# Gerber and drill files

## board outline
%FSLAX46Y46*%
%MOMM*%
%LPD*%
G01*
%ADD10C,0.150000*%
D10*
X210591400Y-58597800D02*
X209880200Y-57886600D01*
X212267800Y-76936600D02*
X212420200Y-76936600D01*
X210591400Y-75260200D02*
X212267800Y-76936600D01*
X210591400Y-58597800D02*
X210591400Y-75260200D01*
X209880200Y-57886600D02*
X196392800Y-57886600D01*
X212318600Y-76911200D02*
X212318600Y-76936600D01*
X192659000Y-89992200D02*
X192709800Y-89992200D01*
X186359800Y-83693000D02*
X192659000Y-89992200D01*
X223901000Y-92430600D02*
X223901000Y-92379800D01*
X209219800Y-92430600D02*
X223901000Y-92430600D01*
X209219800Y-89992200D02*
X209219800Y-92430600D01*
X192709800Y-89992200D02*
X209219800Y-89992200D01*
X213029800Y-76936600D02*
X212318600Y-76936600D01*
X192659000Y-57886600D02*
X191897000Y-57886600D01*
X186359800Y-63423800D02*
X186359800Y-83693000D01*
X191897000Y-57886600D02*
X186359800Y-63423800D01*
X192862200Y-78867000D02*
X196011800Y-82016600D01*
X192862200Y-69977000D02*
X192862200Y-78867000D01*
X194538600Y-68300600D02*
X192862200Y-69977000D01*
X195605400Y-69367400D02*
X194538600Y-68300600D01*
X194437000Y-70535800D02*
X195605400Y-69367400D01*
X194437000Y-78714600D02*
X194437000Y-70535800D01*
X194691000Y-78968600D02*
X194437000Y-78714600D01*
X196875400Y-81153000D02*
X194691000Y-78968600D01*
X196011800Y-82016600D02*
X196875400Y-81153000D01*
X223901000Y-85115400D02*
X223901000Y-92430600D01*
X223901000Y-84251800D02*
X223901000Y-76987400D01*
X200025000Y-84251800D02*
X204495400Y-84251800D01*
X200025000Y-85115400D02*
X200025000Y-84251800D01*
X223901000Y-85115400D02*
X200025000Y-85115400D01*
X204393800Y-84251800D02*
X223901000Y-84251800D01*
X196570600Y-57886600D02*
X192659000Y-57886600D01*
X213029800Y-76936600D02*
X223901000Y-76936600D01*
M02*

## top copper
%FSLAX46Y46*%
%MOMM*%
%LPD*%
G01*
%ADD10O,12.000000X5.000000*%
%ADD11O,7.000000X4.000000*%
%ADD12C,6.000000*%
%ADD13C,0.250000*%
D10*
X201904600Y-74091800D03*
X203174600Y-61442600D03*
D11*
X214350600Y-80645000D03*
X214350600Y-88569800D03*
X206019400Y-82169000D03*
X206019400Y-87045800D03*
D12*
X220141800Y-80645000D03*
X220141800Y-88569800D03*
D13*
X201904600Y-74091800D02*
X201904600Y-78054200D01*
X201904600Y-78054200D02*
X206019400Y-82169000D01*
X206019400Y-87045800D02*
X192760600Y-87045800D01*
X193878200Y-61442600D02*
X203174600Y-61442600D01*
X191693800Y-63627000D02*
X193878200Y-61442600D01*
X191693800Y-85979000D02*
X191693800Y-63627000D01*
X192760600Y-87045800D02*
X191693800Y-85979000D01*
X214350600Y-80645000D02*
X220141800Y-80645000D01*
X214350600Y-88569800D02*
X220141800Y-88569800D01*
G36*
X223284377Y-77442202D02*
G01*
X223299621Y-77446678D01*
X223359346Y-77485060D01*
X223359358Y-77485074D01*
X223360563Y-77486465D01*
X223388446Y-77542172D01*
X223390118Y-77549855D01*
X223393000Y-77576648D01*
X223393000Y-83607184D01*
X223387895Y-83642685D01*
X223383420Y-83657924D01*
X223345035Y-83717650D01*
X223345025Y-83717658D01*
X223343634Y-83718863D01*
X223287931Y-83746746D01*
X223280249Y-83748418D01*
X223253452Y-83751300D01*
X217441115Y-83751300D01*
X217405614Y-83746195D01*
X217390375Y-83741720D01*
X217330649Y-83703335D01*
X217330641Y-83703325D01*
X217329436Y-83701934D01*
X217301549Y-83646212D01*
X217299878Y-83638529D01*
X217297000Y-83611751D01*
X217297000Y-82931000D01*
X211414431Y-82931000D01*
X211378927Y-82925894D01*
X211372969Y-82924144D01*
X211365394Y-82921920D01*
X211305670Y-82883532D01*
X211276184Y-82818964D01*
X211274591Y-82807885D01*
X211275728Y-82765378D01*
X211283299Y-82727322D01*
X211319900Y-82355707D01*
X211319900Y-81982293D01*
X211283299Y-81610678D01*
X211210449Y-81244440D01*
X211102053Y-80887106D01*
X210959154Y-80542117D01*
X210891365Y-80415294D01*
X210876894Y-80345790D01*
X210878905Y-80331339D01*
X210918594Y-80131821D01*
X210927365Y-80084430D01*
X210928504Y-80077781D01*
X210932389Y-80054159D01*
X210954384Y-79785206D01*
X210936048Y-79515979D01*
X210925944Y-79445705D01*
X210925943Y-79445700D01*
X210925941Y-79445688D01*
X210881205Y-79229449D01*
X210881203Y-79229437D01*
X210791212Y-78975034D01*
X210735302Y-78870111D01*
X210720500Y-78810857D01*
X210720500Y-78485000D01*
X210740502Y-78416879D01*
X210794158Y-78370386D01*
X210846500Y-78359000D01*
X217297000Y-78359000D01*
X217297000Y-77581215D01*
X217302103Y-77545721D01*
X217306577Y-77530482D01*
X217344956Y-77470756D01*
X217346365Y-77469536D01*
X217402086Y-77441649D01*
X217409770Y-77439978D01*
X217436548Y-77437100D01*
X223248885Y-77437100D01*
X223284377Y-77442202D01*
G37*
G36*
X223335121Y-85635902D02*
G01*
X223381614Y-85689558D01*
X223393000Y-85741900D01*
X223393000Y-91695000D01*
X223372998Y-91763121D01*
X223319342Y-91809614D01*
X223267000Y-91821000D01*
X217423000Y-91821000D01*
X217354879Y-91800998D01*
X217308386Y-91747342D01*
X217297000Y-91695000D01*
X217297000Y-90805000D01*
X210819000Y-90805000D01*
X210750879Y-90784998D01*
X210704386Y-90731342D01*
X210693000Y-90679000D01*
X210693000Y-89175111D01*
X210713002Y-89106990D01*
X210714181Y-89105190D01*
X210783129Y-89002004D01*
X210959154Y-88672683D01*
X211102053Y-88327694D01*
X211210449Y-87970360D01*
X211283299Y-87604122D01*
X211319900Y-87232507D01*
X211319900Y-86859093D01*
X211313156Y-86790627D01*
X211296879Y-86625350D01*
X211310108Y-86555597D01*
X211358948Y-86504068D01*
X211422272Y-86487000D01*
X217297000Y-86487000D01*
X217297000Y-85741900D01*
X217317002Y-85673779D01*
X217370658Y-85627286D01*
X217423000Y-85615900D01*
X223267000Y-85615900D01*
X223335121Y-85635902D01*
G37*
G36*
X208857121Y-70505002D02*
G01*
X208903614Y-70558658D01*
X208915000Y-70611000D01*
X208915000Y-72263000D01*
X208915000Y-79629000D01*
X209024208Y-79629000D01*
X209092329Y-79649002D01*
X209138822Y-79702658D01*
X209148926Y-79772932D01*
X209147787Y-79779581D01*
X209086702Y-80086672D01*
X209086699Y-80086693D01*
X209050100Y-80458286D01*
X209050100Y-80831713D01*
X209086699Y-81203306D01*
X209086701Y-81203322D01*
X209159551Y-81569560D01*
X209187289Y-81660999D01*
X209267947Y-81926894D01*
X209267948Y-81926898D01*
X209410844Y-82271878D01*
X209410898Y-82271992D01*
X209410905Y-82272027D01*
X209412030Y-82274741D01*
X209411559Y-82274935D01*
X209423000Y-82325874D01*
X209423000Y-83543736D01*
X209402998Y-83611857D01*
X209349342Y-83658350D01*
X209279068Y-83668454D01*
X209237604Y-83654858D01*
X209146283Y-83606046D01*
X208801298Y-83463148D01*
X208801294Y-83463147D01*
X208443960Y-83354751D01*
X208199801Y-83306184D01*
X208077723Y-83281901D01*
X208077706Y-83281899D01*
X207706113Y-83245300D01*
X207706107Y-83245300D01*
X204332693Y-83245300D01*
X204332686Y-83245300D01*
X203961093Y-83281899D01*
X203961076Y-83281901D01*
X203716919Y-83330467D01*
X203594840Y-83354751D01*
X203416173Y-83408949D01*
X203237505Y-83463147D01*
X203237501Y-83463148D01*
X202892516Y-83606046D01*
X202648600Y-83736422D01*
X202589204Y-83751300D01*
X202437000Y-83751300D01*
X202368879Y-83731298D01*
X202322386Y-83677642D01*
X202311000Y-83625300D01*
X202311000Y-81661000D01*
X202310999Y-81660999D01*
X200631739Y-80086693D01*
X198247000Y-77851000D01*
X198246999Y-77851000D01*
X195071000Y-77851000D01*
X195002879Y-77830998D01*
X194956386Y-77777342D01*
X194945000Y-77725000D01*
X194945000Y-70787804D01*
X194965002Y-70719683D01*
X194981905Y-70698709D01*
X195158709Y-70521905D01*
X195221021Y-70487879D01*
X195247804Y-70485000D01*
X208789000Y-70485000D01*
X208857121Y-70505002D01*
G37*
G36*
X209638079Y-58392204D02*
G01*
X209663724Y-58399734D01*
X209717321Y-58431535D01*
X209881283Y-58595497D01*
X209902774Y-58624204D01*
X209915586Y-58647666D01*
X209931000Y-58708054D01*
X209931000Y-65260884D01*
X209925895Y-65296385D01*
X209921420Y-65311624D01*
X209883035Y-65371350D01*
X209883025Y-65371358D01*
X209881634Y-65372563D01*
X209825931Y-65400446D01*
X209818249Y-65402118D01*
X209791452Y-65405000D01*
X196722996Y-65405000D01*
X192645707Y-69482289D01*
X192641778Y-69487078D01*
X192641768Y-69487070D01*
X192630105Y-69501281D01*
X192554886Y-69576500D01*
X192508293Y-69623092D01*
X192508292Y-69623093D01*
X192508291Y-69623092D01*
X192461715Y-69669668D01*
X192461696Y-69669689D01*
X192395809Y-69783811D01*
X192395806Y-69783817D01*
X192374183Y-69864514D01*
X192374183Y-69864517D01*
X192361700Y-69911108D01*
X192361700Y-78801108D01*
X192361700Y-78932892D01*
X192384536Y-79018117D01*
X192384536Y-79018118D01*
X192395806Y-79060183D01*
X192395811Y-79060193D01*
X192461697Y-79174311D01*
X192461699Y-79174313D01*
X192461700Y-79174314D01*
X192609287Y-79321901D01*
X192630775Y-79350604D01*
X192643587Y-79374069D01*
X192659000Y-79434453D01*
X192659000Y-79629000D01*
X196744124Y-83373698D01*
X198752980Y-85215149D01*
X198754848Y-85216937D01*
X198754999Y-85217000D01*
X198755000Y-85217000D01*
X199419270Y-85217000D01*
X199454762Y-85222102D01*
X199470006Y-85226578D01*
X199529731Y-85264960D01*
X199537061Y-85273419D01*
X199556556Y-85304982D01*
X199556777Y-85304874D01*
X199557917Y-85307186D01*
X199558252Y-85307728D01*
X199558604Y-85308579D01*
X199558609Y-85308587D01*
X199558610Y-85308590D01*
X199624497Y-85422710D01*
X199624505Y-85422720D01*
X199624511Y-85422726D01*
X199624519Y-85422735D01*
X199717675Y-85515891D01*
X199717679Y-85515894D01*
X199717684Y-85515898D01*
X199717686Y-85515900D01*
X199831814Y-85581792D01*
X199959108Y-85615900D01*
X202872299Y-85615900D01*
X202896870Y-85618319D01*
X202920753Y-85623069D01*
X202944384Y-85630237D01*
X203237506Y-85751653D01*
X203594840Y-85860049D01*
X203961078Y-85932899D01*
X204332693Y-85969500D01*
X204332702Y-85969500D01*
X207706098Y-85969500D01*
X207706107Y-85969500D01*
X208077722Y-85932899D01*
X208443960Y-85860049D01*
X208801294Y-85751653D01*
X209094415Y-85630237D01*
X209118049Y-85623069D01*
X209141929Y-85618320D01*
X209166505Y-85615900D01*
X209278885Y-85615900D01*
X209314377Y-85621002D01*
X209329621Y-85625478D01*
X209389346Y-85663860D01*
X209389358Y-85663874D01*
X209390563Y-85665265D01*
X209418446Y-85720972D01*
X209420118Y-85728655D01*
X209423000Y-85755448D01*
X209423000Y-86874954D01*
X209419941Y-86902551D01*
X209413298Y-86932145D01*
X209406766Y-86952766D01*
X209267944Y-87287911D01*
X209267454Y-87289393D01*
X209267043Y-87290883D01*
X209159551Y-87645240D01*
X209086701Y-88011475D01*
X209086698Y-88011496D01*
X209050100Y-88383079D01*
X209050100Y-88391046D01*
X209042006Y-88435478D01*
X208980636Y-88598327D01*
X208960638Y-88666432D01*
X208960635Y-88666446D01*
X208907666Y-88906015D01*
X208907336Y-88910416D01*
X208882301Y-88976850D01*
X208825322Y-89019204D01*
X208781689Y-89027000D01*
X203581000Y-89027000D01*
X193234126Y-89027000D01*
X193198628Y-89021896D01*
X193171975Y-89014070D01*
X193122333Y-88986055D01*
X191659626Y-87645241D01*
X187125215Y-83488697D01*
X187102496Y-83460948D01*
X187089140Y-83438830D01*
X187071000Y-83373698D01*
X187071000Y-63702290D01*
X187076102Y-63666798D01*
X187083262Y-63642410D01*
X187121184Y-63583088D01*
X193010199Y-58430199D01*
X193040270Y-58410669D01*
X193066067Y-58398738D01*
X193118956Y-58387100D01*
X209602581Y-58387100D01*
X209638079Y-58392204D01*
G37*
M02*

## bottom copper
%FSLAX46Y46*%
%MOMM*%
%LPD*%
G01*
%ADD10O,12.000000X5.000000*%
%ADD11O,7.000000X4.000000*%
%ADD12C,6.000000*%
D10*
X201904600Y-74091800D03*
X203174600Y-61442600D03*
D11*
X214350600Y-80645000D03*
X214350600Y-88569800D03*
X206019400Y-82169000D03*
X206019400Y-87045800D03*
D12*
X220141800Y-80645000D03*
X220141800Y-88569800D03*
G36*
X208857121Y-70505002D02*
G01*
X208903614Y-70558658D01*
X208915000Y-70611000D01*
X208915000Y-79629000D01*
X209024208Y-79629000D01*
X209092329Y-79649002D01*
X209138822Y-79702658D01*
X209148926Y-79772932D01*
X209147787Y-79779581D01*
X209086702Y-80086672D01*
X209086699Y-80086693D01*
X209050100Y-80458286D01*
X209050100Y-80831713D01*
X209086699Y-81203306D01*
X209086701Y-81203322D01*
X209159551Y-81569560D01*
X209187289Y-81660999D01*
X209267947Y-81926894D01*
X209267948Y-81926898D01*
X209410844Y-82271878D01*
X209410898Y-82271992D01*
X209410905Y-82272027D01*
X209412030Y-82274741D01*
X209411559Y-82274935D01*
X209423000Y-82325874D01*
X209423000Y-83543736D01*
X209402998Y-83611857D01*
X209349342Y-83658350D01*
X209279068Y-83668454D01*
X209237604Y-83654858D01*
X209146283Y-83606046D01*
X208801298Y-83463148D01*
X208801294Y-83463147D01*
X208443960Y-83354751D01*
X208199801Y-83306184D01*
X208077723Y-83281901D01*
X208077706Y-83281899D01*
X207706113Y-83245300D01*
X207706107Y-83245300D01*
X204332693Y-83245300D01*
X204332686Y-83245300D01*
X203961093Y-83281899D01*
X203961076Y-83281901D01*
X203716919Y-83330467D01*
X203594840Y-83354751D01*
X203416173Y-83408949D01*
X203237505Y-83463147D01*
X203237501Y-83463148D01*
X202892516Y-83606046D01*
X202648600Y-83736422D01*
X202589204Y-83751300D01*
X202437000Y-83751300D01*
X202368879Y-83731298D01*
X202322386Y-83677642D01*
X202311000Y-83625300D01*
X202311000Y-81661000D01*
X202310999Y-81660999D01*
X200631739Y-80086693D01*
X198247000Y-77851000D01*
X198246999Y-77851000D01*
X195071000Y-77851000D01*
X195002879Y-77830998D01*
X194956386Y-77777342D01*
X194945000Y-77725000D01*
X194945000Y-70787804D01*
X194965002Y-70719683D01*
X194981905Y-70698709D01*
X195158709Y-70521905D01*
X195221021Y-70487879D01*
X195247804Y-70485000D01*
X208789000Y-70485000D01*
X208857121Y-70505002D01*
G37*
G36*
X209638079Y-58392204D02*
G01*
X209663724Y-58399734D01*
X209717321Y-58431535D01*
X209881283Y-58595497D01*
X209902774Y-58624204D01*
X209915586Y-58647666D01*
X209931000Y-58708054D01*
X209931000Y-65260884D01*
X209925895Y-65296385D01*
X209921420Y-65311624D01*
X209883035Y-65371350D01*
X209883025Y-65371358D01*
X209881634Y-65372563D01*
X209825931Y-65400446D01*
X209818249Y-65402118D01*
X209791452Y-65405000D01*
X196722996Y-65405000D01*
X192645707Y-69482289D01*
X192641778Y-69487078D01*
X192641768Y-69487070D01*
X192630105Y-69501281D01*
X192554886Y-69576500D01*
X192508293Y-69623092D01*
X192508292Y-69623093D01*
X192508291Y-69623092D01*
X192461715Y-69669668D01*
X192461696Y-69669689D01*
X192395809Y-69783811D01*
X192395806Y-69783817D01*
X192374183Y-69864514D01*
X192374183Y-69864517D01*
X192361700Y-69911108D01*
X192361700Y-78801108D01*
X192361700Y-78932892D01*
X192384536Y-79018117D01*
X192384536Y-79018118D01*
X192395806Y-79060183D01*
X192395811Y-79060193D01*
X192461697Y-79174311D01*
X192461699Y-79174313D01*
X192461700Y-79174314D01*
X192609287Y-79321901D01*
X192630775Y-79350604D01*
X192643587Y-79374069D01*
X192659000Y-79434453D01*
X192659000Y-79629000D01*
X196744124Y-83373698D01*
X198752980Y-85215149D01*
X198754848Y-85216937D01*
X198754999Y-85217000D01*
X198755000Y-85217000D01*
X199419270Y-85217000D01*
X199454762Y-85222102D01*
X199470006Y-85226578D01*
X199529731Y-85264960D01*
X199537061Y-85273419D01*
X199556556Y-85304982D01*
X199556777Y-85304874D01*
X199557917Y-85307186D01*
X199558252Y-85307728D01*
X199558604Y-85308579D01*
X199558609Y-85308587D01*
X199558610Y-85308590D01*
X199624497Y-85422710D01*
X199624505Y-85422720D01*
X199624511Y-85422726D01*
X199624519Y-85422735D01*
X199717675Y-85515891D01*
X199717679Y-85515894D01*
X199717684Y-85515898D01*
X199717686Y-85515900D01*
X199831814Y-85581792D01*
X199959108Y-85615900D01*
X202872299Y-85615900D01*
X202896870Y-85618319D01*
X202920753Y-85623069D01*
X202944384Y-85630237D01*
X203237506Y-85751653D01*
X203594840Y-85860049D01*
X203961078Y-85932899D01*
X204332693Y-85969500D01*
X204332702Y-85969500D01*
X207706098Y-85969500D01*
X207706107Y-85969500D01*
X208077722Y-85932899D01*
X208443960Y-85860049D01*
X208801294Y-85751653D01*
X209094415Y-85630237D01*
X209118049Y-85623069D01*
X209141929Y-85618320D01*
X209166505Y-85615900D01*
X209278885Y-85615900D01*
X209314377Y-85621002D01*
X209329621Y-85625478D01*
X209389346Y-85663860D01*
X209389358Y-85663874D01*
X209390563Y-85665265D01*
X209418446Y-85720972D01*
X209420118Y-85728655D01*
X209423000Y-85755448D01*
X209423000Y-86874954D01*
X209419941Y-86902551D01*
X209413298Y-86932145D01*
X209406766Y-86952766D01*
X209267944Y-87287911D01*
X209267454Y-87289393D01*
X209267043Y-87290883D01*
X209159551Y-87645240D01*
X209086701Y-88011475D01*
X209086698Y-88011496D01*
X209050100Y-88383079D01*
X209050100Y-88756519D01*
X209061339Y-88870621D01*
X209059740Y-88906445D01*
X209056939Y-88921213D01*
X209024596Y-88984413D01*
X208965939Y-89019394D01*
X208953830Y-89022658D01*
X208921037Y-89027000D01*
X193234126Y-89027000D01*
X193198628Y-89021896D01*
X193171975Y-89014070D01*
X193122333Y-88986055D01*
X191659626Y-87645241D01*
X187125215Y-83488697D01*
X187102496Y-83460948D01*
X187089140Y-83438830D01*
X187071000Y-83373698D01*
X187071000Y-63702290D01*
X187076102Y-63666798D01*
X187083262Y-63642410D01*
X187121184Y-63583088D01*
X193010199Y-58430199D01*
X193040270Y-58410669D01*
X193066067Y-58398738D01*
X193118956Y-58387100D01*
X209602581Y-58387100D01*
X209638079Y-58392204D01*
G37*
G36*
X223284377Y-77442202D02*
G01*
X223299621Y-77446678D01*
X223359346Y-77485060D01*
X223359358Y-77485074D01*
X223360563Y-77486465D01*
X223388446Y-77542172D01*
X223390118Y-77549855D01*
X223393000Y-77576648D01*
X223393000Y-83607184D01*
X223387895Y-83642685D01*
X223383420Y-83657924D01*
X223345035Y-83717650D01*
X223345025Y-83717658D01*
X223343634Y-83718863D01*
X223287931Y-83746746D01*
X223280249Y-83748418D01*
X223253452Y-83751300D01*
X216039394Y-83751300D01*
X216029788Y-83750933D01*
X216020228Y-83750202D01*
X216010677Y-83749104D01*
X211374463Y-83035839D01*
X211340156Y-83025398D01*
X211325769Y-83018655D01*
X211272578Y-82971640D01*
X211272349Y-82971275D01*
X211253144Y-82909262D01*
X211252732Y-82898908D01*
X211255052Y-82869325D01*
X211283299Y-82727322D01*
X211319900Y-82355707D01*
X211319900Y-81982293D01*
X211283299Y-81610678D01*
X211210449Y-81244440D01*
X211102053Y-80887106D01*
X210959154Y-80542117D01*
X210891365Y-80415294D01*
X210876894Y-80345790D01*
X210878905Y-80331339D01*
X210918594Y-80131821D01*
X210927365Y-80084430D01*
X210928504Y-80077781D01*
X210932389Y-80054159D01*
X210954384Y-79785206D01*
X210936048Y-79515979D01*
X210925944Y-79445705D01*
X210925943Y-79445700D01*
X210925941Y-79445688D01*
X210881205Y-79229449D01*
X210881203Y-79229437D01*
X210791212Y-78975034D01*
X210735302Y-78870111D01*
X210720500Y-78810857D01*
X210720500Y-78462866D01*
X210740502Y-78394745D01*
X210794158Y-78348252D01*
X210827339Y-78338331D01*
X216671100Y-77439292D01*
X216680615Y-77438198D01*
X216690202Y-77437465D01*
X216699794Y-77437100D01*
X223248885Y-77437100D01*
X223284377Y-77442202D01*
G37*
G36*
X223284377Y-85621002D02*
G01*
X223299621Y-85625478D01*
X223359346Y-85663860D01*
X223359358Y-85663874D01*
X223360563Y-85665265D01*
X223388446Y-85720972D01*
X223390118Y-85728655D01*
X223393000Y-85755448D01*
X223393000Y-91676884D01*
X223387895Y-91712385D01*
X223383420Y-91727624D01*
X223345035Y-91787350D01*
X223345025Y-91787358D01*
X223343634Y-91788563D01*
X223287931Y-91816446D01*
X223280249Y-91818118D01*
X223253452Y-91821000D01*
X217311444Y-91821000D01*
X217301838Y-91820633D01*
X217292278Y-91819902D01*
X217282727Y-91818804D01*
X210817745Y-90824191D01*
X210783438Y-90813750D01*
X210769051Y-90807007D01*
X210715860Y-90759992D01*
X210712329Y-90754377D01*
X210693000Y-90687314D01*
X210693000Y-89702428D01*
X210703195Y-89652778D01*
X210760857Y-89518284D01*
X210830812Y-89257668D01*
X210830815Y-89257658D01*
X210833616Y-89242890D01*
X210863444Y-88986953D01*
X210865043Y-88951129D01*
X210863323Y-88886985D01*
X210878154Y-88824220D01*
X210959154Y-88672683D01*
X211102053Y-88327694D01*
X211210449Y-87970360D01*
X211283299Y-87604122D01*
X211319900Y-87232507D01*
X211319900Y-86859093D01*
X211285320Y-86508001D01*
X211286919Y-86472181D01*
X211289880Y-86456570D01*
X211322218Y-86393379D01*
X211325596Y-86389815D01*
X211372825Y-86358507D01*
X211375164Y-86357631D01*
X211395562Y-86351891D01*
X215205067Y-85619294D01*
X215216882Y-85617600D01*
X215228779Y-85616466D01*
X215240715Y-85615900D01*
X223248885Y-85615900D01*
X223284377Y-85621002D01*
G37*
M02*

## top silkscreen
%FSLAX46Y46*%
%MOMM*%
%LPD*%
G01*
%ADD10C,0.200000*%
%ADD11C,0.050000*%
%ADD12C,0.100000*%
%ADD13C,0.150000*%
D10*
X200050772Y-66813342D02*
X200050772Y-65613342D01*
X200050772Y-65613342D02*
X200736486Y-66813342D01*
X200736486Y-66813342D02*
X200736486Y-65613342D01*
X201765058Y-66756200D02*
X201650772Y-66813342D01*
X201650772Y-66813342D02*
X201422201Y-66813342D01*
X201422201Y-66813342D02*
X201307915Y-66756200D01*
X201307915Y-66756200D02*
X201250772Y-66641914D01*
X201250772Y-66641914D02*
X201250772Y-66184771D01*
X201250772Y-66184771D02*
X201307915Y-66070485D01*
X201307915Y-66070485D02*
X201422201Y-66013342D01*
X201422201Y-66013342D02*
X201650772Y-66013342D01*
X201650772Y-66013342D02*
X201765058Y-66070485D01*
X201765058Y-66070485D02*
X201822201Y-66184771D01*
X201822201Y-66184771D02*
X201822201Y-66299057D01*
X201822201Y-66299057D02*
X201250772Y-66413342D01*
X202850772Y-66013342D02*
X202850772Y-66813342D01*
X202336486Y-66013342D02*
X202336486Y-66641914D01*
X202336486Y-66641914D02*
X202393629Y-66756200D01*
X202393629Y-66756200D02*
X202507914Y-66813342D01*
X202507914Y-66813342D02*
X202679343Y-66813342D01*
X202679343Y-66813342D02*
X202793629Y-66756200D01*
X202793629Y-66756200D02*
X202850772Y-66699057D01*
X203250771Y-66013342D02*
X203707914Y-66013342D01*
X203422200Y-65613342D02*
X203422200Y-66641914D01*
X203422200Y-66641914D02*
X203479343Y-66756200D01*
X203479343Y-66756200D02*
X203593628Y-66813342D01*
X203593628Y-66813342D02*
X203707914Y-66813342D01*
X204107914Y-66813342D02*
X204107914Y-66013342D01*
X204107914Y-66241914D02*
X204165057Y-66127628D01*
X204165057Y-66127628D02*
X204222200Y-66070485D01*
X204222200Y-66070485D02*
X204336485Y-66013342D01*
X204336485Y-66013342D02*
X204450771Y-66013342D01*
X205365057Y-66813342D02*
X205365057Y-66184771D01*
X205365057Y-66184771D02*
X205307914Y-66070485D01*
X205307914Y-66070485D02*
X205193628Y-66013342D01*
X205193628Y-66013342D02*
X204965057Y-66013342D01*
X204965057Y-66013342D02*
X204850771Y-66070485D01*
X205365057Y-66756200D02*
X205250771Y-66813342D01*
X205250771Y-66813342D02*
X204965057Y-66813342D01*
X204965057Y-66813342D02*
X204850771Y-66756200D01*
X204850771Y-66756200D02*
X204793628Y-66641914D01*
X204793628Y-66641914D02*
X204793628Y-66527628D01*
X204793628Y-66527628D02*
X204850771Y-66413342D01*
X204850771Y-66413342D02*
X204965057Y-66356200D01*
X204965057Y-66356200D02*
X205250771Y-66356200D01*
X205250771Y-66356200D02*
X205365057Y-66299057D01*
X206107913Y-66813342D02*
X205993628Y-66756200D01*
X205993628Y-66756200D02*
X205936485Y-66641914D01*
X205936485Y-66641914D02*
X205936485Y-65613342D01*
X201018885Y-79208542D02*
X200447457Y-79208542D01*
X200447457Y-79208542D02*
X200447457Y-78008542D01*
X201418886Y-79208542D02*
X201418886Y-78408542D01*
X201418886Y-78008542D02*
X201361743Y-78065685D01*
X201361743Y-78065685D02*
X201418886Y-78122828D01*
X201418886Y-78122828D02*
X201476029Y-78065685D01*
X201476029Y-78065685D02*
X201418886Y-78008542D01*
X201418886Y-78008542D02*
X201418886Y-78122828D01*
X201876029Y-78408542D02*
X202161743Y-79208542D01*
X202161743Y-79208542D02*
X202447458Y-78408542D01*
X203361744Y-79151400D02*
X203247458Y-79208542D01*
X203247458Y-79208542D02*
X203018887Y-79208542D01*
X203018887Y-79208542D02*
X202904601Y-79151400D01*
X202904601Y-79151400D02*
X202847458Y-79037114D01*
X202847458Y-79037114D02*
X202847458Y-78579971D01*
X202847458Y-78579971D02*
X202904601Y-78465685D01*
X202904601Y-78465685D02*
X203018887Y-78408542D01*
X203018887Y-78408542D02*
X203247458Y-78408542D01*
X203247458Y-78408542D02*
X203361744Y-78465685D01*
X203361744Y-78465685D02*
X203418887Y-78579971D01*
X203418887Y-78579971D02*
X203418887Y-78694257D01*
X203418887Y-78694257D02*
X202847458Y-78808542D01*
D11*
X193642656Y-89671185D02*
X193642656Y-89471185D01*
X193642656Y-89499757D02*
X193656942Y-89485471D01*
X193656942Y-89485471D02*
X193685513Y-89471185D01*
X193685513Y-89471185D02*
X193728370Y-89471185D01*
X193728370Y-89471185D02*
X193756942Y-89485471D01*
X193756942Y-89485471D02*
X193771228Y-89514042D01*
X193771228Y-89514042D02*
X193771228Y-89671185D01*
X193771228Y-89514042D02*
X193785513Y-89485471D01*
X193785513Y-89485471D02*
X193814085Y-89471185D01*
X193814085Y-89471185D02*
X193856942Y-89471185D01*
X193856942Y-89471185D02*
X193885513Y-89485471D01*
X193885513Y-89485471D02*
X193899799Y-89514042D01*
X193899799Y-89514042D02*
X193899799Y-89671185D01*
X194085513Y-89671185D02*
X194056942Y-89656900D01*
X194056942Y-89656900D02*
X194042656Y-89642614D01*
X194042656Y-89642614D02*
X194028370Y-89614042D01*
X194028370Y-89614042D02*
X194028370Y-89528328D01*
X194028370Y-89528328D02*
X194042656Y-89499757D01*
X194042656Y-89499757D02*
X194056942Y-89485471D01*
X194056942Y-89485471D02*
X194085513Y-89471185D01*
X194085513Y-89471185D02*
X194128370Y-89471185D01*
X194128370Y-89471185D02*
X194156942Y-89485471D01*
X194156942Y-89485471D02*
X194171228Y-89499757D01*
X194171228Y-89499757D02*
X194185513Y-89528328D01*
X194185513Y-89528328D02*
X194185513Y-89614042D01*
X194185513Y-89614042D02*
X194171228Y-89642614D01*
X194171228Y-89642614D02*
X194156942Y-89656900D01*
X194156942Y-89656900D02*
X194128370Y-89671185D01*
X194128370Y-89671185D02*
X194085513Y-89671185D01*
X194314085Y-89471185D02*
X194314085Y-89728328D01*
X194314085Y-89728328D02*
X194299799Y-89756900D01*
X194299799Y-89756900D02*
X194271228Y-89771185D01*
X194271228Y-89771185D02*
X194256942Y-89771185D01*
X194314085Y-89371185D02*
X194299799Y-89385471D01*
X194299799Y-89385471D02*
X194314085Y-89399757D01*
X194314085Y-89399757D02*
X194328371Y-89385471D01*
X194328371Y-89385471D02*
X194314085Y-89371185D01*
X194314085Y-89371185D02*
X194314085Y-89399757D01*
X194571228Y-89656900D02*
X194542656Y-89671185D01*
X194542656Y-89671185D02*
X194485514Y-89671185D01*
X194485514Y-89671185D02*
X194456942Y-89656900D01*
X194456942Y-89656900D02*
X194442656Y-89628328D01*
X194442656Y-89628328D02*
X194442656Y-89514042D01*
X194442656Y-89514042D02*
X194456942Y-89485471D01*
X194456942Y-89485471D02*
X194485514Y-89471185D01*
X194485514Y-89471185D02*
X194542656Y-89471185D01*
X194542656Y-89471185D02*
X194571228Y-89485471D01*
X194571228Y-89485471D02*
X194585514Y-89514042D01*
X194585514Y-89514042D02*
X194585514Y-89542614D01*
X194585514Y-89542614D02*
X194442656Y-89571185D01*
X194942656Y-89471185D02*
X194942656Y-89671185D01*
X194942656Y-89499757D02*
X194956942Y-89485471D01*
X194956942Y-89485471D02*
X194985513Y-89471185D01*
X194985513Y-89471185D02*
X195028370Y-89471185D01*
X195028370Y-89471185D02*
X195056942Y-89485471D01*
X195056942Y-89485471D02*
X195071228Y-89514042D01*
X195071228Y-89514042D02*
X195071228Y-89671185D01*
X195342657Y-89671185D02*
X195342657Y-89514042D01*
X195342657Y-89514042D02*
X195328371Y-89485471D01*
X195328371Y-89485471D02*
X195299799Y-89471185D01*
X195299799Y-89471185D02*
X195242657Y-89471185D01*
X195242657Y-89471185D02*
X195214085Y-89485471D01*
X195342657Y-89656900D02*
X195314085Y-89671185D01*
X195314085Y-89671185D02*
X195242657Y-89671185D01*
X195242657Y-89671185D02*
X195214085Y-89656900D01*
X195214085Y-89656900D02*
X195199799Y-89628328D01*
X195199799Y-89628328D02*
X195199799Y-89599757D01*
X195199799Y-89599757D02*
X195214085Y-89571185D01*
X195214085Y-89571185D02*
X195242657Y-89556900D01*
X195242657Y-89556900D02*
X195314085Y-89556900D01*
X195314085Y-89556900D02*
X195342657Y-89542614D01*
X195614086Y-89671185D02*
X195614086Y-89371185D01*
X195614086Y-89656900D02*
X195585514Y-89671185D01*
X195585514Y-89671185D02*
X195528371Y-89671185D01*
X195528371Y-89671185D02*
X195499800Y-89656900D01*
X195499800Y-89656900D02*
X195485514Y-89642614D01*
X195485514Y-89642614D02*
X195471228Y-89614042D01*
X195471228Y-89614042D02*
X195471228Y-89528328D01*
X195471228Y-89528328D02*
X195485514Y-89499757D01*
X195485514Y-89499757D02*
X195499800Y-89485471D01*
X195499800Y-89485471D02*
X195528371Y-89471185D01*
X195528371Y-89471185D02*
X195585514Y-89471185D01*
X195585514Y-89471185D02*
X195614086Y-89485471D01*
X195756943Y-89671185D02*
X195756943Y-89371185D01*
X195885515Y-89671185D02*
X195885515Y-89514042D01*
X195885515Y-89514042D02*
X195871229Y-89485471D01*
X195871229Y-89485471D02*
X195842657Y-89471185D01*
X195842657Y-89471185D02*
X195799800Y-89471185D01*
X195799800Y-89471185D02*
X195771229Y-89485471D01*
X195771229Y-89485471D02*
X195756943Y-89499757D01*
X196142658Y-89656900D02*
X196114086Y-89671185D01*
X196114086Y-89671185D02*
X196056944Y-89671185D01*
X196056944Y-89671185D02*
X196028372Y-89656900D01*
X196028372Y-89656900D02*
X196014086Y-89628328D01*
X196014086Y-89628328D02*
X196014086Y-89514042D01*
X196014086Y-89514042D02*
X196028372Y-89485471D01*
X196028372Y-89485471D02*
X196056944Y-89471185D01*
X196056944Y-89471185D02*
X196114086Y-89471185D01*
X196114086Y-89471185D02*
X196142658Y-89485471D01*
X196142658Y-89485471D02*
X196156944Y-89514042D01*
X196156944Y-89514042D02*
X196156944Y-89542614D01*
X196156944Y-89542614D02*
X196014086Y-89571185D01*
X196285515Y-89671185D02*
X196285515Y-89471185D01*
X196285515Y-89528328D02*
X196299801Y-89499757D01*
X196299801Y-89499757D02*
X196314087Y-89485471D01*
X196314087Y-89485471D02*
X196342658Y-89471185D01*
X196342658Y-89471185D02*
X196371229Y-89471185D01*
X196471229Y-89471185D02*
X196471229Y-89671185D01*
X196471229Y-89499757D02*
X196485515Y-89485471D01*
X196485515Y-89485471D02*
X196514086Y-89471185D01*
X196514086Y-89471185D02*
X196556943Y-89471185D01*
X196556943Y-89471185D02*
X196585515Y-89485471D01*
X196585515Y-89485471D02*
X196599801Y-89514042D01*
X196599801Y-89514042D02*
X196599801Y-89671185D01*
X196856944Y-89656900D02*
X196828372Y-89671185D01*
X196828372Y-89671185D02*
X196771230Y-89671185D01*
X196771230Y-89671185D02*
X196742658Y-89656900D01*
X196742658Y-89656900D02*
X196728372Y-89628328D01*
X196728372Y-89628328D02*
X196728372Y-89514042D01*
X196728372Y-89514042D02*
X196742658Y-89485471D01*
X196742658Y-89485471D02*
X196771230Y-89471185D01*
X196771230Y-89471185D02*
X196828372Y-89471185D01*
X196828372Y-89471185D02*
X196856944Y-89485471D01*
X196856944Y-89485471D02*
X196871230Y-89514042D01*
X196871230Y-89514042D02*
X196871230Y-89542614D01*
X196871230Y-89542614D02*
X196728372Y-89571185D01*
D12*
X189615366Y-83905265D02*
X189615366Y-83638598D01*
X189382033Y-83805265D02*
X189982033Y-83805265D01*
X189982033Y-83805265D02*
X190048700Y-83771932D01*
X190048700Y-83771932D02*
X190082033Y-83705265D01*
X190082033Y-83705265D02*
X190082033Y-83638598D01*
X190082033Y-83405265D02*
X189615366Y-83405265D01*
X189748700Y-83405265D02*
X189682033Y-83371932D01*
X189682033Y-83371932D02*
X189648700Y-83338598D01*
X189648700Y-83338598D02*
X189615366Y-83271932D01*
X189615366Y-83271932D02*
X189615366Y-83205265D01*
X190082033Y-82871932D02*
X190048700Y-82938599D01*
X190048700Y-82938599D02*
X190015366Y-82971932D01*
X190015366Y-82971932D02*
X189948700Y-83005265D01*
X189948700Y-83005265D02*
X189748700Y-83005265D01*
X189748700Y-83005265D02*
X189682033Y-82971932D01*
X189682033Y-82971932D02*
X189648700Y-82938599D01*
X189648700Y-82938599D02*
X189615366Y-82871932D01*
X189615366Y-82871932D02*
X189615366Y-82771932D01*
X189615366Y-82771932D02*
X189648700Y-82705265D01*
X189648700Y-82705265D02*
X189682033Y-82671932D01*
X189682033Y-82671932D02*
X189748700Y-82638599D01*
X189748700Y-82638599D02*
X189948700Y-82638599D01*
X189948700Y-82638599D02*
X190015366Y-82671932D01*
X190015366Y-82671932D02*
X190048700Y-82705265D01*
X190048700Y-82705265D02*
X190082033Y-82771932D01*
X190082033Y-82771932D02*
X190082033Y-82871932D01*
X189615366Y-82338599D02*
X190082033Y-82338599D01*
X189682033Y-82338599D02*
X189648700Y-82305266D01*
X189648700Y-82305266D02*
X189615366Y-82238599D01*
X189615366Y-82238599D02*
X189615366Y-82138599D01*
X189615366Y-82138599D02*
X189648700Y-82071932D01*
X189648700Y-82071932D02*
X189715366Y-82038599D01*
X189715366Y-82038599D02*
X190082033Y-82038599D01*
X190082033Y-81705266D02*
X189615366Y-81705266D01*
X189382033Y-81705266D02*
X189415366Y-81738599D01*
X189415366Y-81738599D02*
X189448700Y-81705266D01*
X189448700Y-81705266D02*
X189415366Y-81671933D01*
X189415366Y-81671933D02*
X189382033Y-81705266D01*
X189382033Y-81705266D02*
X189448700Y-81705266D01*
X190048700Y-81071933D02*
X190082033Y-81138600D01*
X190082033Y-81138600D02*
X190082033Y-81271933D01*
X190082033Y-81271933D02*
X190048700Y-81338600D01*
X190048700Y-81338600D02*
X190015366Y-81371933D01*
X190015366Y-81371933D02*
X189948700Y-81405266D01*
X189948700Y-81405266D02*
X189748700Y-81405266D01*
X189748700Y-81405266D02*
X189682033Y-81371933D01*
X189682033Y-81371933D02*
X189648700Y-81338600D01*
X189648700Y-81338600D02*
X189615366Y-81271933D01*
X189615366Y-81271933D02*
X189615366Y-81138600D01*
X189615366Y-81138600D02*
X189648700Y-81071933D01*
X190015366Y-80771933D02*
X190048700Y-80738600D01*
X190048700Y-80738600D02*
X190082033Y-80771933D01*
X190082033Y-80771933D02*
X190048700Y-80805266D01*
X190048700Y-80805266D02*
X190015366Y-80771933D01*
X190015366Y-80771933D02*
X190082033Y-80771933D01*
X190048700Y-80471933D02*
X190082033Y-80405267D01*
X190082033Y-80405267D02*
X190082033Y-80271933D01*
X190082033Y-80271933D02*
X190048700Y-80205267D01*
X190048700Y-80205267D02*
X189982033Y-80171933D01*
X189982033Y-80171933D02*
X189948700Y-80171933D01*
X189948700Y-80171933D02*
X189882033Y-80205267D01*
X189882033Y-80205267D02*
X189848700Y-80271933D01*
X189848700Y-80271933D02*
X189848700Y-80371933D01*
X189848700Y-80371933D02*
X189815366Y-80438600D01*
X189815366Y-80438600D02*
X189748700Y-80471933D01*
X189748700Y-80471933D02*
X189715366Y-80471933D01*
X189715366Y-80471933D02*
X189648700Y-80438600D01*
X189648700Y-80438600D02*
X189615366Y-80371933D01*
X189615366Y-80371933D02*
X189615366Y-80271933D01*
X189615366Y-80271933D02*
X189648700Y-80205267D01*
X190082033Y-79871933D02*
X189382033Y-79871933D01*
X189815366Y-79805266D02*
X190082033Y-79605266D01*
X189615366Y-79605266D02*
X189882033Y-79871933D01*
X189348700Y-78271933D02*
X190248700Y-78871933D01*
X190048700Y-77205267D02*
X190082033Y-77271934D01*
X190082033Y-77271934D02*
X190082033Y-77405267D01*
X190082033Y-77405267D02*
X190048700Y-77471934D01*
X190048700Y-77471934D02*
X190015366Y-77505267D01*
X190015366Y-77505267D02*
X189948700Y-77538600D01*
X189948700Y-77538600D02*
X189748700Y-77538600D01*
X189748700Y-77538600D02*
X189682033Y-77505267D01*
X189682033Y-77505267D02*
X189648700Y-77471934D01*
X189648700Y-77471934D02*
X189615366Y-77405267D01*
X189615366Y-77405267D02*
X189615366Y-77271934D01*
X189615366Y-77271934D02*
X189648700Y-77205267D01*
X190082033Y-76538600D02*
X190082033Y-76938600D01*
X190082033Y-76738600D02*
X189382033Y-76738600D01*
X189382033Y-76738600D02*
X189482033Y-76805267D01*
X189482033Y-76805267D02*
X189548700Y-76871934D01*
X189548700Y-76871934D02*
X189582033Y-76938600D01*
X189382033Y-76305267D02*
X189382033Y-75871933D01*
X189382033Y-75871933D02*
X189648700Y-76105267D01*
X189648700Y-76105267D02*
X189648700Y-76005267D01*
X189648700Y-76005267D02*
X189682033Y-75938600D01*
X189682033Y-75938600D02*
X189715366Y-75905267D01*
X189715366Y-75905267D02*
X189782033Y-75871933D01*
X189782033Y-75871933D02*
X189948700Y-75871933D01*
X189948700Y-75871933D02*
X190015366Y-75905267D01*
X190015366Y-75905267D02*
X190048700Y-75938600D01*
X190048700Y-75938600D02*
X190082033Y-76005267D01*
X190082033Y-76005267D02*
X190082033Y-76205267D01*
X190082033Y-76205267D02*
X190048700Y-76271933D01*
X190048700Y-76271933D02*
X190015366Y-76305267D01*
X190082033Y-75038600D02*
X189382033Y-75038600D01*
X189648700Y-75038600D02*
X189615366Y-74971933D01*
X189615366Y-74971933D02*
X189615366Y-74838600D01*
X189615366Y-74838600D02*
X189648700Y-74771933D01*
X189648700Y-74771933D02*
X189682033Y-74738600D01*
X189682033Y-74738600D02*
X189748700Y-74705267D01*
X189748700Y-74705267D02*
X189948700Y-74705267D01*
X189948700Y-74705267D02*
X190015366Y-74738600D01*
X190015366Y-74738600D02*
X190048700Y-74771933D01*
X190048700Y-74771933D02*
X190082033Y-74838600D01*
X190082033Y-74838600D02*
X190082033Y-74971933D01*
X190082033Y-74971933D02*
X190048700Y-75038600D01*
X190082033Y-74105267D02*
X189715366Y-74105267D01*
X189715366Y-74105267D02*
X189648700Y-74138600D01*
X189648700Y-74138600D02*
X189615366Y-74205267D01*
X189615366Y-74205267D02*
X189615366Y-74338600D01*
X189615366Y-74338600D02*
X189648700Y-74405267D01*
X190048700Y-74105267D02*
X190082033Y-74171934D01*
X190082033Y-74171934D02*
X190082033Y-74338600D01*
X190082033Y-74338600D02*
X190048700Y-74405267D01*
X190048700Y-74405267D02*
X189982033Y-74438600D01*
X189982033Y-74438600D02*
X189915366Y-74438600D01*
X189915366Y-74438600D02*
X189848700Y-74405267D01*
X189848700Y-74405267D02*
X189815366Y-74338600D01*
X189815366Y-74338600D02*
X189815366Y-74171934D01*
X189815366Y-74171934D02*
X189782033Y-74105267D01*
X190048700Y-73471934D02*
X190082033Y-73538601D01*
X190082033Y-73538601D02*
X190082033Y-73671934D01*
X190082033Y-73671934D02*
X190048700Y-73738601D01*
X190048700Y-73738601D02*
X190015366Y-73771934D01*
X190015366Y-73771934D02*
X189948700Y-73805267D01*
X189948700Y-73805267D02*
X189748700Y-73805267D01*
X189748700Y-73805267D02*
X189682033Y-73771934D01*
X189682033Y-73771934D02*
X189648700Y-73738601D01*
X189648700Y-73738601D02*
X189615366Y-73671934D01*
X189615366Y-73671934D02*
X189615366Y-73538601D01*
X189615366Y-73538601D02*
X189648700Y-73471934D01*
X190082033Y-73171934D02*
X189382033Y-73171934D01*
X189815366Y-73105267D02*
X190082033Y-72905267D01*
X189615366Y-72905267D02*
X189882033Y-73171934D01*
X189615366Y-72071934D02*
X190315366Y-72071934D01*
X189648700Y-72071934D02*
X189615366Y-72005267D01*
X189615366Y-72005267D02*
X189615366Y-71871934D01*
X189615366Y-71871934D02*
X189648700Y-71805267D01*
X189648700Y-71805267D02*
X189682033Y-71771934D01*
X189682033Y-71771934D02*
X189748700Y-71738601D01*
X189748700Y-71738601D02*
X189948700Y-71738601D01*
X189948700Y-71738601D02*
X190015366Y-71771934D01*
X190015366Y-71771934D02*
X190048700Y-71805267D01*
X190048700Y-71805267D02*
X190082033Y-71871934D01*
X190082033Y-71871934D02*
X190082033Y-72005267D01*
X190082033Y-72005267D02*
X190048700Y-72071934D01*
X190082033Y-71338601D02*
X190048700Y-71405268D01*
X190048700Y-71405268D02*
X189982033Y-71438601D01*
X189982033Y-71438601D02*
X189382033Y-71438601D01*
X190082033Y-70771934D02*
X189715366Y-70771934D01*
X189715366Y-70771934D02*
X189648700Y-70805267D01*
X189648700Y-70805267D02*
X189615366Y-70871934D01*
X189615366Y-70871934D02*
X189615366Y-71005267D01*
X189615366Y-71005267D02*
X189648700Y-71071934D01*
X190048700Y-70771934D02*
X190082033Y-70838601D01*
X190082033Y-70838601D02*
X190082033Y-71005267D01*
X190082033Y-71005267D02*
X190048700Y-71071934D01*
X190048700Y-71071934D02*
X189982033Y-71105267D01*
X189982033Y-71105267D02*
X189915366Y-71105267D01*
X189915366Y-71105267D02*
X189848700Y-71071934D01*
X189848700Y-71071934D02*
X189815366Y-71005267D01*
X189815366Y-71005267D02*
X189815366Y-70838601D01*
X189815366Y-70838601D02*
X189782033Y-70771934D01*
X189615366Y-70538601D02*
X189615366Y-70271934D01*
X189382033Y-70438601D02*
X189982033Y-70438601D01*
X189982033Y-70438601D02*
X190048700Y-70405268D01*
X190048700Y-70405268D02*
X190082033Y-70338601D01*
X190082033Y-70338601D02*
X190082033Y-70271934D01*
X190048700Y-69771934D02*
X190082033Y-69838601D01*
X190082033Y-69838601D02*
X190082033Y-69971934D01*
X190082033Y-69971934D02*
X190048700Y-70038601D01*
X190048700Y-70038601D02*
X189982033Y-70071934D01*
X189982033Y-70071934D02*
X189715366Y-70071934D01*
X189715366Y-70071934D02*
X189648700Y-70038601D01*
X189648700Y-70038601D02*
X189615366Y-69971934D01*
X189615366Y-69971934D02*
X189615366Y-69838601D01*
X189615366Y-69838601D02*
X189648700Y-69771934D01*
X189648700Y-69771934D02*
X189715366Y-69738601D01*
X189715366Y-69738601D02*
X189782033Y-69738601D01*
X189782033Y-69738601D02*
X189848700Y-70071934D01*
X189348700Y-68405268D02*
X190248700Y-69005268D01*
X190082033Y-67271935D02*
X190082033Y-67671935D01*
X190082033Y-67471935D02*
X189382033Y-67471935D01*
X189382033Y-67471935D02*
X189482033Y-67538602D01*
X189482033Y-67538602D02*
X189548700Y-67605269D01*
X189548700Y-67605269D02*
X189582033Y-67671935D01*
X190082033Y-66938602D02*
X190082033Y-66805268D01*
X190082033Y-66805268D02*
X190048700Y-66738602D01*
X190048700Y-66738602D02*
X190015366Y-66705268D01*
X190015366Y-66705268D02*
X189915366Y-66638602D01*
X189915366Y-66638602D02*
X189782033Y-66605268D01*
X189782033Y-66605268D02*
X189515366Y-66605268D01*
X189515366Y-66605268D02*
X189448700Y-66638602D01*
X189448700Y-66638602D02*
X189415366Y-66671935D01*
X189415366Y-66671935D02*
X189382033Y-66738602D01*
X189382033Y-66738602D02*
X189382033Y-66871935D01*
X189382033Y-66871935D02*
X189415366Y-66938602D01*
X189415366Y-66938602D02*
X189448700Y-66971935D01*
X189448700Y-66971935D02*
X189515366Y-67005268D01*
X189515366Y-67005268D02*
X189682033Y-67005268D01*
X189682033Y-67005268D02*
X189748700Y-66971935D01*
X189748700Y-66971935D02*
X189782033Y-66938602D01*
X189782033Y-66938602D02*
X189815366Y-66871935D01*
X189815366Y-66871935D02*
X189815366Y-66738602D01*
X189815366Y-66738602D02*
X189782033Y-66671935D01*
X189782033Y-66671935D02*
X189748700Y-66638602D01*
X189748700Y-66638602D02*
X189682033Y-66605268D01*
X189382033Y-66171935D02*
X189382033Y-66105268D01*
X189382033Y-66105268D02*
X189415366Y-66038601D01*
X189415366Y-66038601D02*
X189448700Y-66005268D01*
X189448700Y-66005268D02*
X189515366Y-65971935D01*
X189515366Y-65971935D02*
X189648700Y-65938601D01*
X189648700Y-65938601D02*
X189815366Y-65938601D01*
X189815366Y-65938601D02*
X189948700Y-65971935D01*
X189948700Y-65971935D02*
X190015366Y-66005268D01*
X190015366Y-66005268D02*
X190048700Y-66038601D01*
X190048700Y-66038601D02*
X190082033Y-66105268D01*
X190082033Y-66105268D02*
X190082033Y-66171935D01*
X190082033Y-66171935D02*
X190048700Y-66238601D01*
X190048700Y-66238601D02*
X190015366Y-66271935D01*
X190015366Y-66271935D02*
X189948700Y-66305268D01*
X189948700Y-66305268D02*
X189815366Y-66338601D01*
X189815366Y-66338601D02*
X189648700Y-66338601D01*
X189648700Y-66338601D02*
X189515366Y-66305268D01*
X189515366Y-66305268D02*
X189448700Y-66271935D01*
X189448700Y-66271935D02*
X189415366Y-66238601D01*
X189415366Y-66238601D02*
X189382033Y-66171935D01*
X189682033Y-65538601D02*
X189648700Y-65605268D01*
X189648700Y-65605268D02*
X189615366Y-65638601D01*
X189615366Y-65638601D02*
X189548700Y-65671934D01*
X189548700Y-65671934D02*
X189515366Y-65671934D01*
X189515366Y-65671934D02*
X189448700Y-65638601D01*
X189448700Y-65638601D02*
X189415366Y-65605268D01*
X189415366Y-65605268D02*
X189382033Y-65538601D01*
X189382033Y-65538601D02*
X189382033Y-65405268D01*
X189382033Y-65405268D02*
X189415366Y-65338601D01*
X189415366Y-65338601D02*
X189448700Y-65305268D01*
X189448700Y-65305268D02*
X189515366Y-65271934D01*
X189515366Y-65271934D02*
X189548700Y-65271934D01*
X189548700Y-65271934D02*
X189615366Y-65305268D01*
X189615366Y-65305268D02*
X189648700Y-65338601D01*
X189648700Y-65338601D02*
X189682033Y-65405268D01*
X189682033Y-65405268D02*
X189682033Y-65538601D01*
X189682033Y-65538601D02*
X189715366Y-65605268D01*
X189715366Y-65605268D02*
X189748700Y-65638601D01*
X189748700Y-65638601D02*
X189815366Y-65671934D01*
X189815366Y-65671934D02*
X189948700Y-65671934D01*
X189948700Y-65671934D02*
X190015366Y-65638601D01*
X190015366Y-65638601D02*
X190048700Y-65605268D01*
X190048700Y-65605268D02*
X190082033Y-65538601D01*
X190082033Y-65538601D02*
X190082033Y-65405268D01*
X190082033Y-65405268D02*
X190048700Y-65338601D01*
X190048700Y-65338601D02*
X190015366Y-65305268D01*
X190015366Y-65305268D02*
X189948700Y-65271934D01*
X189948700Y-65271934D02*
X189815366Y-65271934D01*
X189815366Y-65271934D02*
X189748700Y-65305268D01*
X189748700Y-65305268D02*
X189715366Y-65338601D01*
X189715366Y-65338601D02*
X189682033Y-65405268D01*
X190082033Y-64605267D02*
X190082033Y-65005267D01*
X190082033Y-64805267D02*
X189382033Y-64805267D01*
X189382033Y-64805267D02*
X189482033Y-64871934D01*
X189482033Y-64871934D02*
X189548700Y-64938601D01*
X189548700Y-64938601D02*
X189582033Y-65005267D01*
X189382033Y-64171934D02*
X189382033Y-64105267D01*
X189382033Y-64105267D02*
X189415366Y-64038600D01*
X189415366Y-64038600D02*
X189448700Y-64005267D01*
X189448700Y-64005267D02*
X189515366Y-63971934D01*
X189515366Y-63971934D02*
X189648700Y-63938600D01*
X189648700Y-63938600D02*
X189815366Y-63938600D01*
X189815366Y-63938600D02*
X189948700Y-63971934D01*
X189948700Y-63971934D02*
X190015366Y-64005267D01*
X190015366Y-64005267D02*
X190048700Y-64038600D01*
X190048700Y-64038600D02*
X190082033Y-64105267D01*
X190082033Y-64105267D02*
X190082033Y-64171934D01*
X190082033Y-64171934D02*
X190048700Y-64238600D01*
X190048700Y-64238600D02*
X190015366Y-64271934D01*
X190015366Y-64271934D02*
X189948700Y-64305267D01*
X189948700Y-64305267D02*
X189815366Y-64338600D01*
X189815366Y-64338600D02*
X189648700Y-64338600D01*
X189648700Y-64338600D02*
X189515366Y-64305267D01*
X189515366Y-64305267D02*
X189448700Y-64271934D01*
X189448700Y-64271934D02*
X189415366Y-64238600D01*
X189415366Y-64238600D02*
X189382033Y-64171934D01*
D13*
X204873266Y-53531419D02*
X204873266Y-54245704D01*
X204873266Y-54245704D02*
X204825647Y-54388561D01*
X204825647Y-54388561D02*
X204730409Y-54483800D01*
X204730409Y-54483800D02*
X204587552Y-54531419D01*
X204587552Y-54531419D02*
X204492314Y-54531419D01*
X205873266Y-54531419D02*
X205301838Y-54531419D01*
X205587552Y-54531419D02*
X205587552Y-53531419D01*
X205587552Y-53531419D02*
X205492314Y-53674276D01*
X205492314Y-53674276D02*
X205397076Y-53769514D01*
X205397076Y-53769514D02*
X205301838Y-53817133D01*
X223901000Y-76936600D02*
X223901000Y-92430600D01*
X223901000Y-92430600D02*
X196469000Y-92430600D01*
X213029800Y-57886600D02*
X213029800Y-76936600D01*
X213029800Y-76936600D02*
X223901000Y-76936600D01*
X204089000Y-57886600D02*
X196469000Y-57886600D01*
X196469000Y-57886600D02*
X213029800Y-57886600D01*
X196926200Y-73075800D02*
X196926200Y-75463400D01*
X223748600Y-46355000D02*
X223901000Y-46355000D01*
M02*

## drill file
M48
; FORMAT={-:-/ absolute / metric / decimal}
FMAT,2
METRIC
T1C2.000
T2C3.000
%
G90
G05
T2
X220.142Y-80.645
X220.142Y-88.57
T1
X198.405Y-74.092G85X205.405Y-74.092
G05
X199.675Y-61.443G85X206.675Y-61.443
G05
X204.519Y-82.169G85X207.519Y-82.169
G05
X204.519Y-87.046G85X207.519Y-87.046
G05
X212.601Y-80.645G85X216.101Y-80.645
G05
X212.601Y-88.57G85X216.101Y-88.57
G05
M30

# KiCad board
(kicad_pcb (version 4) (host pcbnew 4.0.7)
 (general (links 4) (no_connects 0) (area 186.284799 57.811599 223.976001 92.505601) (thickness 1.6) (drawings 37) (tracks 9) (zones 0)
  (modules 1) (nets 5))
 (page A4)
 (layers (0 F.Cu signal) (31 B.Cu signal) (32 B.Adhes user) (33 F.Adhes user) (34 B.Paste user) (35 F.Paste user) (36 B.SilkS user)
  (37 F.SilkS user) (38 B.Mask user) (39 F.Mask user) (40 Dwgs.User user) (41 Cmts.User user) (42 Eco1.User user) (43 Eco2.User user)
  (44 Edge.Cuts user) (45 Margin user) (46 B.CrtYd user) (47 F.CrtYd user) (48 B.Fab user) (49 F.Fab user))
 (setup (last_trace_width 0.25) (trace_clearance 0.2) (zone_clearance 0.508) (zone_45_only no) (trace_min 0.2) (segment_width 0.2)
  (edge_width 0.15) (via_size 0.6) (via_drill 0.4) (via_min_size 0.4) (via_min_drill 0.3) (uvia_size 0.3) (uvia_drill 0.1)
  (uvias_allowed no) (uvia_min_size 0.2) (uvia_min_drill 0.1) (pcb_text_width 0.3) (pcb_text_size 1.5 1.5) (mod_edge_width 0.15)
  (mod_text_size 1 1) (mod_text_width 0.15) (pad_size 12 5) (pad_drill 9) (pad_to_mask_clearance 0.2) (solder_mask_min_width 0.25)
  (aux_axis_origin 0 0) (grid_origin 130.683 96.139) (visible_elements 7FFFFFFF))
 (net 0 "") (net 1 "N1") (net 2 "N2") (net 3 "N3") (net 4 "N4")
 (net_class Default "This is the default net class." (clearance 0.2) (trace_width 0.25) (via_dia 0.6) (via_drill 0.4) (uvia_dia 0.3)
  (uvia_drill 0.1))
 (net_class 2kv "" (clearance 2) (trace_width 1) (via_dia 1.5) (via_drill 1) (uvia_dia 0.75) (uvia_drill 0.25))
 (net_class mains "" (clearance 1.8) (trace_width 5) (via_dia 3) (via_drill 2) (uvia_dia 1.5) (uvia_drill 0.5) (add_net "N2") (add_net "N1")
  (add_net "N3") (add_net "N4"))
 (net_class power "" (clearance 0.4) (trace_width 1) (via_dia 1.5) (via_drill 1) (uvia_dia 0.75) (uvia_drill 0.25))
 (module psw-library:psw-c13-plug (layer F.Cu) (at 196.469 46.355)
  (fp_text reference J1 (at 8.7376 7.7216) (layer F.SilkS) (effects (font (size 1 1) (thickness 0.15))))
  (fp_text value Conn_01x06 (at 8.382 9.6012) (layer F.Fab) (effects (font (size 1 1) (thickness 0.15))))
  (fp_line (start 27.432 30.5816) (end 27.432 46.0756) (layer F.SilkS) (width 0.15))
  (fp_line (start 27.432 46.0756) (end 0 46.0756) (layer F.SilkS) (width 0.15))
  (fp_line (start 16.5608 11.5316) (end 16.5608 30.5816) (layer F.SilkS) (width 0.15))
  (fp_line (start 16.5608 30.5816) (end 27.432 30.5816) (layer F.SilkS) (width 0.15))
  (fp_line (start 7.62 11.5316) (end 0 11.5316) (layer F.SilkS) (width 0.15))
  (fp_line (start 0 11.5316) (end 16.5608 11.5316) (layer F.SilkS) (width 0.15))
  (fp_line (start 0.4572 26.7208) (end 0.4572 29.1084) (layer F.SilkS) (width 0.15))
  (fp_line (start 27.2796 0) (end 27.432 0) (layer F.SilkS) (width 0.15))
  (pad 2 thru_hole oval (at 5.4356 27.7368) (size 12 5) (drill oval 9 2) (layers *.Cu *.Mask) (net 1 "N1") (zone_connect 2))
  (pad 1 thru_hole oval (at 6.7056 15.0876) (size 12 5) (drill oval 9 2) (layers *.Cu *.Mask) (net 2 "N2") (zone_connect 2))
  (pad 5 thru_hole oval (at 17.8816 34.29) (size 7 4) (drill oval 5.5 2) (layers *.Cu *.Mask) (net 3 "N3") (zone_connect 2))
  (pad 6 thru_hole oval (at 17.8816 42.2148) (size 7 4) (drill oval 5.5 2) (layers *.Cu *.Mask) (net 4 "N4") (zone_connect 2))
  (pad 3 thru_hole oval (at 9.5504 35.814) (size 7 4) (drill oval 5 2) (layers *.Cu *.Mask) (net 1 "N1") (zone_connect 2))
  (pad 4 thru_hole oval (at 9.5504 40.6908) (size 7 4) (drill oval 5 2) (layers *.Cu *.Mask) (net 2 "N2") (zone_connect 2))
  (pad 5 thru_hole circle (at 23.6728 34.29) (size 6 6) (drill 3) (layers *.Cu *.Mask) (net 3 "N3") (zone_connect 2))
  (pad 6 thru_hole circle (at 23.6728 42.2148) (size 6 6) (drill 3) (layers *.Cu *.Mask) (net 4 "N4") (zone_connect 2)))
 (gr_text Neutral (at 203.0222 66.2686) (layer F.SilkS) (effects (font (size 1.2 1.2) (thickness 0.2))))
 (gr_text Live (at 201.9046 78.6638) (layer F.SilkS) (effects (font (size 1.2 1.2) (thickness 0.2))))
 (gr_line (start 210.5914 58.5978) (end 209.8802 57.8866) (angle 90) (layer Edge.Cuts) (width 0.15))
 (gr_line (start 212.2678 76.9366) (end 212.4202 76.9366) (angle 90) (layer Edge.Cuts) (width 0.15))
 (gr_line (start 210.5914 75.2602) (end 212.2678 76.9366) (angle 90) (layer Edge.Cuts) (width 0.15))
 (gr_line (start 210.5914 58.5978) (end 210.5914 75.2602) (angle 90) (layer Edge.Cuts) (width 0.15))
 (gr_line (start 209.8802 57.8866) (end 196.3928 57.8866) (angle 90) (layer Edge.Cuts) (width 0.15))
 (gr_line (start 212.3186 76.9112) (end 212.3186 76.9366) (angle 90) (layer Edge.Cuts) (width 0.15))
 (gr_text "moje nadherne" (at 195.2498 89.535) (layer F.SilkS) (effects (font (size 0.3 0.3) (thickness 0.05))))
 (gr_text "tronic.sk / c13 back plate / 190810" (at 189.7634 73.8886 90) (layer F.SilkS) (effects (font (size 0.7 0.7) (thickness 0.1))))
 (gr_line (start 192.659 89.9922) (end 192.7098 89.9922) (angle 90) (layer Edge.Cuts) (width 0.15))
 (gr_line (start 186.3598 83.693) (end 192.659 89.9922) (angle 90) (layer Edge.Cuts) (width 0.15))
 (gr_line (start 223.901 92.4306) (end 223.901 92.3798) (angle 90) (layer Edge.Cuts) (width 0.15))
 (gr_line (start 209.2198 92.4306) (end 223.901 92.4306) (angle 90) (layer Edge.Cuts) (width 0.15))
 (gr_line (start 209.2198 89.9922) (end 209.2198 92.4306) (angle 90) (layer Edge.Cuts) (width 0.15))
 (gr_line (start 192.7098 89.9922) (end 209.2198 89.9922) (angle 90) (layer Edge.Cuts) (width 0.15))
 (gr_line (start 213.0298 76.9366) (end 212.3186 76.9366) (angle 90) (layer Edge.Cuts) (width 0.15))
 (gr_line (start 192.659 57.8866) (end 191.897 57.8866) (angle 90) (layer Edge.Cuts) (width 0.15))
 (gr_line (start 186.3598 63.4238) (end 186.3598 83.693) (angle 90) (layer Edge.Cuts) (width 0.15))
 (gr_line (start 191.897 57.8866) (end 186.3598 63.4238) (angle 90) (layer Edge.Cuts) (width 0.15))
 (gr_line (start 192.8622 78.867) (end 196.0118 82.0166) (angle 90) (layer Edge.Cuts) (width 0.15))
 (gr_line (start 192.8622 69.977) (end 192.8622 78.867) (angle 90) (layer Edge.Cuts) (width 0.15))
 (gr_line (start 194.5386 68.3006) (end 192.8622 69.977) (angle 90) (layer Edge.Cuts) (width 0.15))
 (gr_line (start 195.6054 69.3674) (end 194.5386 68.3006) (angle 90) (layer Edge.Cuts) (width 0.15))
 (gr_line (start 194.437 70.5358) (end 195.6054 69.3674) (angle 90) (layer Edge.Cuts) (width 0.15))
 (gr_line (start 194.437 78.7146) (end 194.437 70.5358) (angle 90) (layer Edge.Cuts) (width 0.15))
 (gr_line (start 194.691 78.9686) (end 194.437 78.7146) (angle 90) (layer Edge.Cuts) (width 0.15))
 (gr_line (start 196.8754 81.153) (end 194.691 78.9686) (angle 90) (layer Edge.Cuts) (width 0.15))
 (gr_line (start 196.0118 82.0166) (end 196.8754 81.153) (angle 90) (layer Edge.Cuts) (width 0.15))
 (gr_line (start 223.901 85.1154) (end 223.901 92.4306) (angle 90) (layer Edge.Cuts) (width 0.15))
 (gr_line (start 223.901 84.2518) (end 223.901 76.9874) (angle 90) (layer Edge.Cuts) (width 0.15))
 (gr_line (start 200.025 84.2518) (end 204.4954 84.2518) (angle 90) (layer Edge.Cuts) (width 0.15))
 (gr_line (start 200.025 85.1154) (end 200.025 84.2518) (angle 90) (layer Edge.Cuts) (width 0.15))
 (gr_line (start 223.901 85.1154) (end 200.025 85.1154) (angle 90) (layer Edge.Cuts) (width 0.15))
 (gr_line (start 204.3938 84.2518) (end 223.901 84.2518) (angle 90) (layer Edge.Cuts) (width 0.15))
 (gr_line (start 196.5706 57.8866) (end 192.659 57.8866) (angle 90) (layer Edge.Cuts) (width 0.15))
 (gr_line (start 213.0298 76.9366) (end 223.901 76.9366) (angle 90) (layer Edge.Cuts) (width 0.15))
 (segment (start 201.9046 74.0918) (end 201.9046 78.0542) (width 0.25) (layer F.Cu) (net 1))
 (segment (start 201.9046 78.0542) (end 206.0194 82.169) (width 0.25) (layer F.Cu) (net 1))
 (segment (start 206.0194 87.0458) (end 192.7606 87.0458) (width 0.25) (layer F.Cu) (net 2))
 (segment (start 193.8782 61.4426) (end 203.1746 61.4426) (width 0.25) (layer F.Cu) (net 2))
 (segment (start 191.6938 63.627) (end 193.8782 61.4426) (width 0.25) (layer F.Cu) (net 2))
 (segment (start 191.6938 85.979) (end 191.6938 63.627) (width 0.25) (layer F.Cu) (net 2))
 (segment (start 192.7606 87.0458) (end 191.6938 85.979) (width 0.25) (layer F.Cu) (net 2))
 (segment (start 214.3506 80.645) (end 220.1418 80.645) (width 0.25) (layer F.Cu) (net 3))
 (segment (start 214.3506 88.5698) (end 220.1418 88.5698) (width 0.25) (layer F.Cu) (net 4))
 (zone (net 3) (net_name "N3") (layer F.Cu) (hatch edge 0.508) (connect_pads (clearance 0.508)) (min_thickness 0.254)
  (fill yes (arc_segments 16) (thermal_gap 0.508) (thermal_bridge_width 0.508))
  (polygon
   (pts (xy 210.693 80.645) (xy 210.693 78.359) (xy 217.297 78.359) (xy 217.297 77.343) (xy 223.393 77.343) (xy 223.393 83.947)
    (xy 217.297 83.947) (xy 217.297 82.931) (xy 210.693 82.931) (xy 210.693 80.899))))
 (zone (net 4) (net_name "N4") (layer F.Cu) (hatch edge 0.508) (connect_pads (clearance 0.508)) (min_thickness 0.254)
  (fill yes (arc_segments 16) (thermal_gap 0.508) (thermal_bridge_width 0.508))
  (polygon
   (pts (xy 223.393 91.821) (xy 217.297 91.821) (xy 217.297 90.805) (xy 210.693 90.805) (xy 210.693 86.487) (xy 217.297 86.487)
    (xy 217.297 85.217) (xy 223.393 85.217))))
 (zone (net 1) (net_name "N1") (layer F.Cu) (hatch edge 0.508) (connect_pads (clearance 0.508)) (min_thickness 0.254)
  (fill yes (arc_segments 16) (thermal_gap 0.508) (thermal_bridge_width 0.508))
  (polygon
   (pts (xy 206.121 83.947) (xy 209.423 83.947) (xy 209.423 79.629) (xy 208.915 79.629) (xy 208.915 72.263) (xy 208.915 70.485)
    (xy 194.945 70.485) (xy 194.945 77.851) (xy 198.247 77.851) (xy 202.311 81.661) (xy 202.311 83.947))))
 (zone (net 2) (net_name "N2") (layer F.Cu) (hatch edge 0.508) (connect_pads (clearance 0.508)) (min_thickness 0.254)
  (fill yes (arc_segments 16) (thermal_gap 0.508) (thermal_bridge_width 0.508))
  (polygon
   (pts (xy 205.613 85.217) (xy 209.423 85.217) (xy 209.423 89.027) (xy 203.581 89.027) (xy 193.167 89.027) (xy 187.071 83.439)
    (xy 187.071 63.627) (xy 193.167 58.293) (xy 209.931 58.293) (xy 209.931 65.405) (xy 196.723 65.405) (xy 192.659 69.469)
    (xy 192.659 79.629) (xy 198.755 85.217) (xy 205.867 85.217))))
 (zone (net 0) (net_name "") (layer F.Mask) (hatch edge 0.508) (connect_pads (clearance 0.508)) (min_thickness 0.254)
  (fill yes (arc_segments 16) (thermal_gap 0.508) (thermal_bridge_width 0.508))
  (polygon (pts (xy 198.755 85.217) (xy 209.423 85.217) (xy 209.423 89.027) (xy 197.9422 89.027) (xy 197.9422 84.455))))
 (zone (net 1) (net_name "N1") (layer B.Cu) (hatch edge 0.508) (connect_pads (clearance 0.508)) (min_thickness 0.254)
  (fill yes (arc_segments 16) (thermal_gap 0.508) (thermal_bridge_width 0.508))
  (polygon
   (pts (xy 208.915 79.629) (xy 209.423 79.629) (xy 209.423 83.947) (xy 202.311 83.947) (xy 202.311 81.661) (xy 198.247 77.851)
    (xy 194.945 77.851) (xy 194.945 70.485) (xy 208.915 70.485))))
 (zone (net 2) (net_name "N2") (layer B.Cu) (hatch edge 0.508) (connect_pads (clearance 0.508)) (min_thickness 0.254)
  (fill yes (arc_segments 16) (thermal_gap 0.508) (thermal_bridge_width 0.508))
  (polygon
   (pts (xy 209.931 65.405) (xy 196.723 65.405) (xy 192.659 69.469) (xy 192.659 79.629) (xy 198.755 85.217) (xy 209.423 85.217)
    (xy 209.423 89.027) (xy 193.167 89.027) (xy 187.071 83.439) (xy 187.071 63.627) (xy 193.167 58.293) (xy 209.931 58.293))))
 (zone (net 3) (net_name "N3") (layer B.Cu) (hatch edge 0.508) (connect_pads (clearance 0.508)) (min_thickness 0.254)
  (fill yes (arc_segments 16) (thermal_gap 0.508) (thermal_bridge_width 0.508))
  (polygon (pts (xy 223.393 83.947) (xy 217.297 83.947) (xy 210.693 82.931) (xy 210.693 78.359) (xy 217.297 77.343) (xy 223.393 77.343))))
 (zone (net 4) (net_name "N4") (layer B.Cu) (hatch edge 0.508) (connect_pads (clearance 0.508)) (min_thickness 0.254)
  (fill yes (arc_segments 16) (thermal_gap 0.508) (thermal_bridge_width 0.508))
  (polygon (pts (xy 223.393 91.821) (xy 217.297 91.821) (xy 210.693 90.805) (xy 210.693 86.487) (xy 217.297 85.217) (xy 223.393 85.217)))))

